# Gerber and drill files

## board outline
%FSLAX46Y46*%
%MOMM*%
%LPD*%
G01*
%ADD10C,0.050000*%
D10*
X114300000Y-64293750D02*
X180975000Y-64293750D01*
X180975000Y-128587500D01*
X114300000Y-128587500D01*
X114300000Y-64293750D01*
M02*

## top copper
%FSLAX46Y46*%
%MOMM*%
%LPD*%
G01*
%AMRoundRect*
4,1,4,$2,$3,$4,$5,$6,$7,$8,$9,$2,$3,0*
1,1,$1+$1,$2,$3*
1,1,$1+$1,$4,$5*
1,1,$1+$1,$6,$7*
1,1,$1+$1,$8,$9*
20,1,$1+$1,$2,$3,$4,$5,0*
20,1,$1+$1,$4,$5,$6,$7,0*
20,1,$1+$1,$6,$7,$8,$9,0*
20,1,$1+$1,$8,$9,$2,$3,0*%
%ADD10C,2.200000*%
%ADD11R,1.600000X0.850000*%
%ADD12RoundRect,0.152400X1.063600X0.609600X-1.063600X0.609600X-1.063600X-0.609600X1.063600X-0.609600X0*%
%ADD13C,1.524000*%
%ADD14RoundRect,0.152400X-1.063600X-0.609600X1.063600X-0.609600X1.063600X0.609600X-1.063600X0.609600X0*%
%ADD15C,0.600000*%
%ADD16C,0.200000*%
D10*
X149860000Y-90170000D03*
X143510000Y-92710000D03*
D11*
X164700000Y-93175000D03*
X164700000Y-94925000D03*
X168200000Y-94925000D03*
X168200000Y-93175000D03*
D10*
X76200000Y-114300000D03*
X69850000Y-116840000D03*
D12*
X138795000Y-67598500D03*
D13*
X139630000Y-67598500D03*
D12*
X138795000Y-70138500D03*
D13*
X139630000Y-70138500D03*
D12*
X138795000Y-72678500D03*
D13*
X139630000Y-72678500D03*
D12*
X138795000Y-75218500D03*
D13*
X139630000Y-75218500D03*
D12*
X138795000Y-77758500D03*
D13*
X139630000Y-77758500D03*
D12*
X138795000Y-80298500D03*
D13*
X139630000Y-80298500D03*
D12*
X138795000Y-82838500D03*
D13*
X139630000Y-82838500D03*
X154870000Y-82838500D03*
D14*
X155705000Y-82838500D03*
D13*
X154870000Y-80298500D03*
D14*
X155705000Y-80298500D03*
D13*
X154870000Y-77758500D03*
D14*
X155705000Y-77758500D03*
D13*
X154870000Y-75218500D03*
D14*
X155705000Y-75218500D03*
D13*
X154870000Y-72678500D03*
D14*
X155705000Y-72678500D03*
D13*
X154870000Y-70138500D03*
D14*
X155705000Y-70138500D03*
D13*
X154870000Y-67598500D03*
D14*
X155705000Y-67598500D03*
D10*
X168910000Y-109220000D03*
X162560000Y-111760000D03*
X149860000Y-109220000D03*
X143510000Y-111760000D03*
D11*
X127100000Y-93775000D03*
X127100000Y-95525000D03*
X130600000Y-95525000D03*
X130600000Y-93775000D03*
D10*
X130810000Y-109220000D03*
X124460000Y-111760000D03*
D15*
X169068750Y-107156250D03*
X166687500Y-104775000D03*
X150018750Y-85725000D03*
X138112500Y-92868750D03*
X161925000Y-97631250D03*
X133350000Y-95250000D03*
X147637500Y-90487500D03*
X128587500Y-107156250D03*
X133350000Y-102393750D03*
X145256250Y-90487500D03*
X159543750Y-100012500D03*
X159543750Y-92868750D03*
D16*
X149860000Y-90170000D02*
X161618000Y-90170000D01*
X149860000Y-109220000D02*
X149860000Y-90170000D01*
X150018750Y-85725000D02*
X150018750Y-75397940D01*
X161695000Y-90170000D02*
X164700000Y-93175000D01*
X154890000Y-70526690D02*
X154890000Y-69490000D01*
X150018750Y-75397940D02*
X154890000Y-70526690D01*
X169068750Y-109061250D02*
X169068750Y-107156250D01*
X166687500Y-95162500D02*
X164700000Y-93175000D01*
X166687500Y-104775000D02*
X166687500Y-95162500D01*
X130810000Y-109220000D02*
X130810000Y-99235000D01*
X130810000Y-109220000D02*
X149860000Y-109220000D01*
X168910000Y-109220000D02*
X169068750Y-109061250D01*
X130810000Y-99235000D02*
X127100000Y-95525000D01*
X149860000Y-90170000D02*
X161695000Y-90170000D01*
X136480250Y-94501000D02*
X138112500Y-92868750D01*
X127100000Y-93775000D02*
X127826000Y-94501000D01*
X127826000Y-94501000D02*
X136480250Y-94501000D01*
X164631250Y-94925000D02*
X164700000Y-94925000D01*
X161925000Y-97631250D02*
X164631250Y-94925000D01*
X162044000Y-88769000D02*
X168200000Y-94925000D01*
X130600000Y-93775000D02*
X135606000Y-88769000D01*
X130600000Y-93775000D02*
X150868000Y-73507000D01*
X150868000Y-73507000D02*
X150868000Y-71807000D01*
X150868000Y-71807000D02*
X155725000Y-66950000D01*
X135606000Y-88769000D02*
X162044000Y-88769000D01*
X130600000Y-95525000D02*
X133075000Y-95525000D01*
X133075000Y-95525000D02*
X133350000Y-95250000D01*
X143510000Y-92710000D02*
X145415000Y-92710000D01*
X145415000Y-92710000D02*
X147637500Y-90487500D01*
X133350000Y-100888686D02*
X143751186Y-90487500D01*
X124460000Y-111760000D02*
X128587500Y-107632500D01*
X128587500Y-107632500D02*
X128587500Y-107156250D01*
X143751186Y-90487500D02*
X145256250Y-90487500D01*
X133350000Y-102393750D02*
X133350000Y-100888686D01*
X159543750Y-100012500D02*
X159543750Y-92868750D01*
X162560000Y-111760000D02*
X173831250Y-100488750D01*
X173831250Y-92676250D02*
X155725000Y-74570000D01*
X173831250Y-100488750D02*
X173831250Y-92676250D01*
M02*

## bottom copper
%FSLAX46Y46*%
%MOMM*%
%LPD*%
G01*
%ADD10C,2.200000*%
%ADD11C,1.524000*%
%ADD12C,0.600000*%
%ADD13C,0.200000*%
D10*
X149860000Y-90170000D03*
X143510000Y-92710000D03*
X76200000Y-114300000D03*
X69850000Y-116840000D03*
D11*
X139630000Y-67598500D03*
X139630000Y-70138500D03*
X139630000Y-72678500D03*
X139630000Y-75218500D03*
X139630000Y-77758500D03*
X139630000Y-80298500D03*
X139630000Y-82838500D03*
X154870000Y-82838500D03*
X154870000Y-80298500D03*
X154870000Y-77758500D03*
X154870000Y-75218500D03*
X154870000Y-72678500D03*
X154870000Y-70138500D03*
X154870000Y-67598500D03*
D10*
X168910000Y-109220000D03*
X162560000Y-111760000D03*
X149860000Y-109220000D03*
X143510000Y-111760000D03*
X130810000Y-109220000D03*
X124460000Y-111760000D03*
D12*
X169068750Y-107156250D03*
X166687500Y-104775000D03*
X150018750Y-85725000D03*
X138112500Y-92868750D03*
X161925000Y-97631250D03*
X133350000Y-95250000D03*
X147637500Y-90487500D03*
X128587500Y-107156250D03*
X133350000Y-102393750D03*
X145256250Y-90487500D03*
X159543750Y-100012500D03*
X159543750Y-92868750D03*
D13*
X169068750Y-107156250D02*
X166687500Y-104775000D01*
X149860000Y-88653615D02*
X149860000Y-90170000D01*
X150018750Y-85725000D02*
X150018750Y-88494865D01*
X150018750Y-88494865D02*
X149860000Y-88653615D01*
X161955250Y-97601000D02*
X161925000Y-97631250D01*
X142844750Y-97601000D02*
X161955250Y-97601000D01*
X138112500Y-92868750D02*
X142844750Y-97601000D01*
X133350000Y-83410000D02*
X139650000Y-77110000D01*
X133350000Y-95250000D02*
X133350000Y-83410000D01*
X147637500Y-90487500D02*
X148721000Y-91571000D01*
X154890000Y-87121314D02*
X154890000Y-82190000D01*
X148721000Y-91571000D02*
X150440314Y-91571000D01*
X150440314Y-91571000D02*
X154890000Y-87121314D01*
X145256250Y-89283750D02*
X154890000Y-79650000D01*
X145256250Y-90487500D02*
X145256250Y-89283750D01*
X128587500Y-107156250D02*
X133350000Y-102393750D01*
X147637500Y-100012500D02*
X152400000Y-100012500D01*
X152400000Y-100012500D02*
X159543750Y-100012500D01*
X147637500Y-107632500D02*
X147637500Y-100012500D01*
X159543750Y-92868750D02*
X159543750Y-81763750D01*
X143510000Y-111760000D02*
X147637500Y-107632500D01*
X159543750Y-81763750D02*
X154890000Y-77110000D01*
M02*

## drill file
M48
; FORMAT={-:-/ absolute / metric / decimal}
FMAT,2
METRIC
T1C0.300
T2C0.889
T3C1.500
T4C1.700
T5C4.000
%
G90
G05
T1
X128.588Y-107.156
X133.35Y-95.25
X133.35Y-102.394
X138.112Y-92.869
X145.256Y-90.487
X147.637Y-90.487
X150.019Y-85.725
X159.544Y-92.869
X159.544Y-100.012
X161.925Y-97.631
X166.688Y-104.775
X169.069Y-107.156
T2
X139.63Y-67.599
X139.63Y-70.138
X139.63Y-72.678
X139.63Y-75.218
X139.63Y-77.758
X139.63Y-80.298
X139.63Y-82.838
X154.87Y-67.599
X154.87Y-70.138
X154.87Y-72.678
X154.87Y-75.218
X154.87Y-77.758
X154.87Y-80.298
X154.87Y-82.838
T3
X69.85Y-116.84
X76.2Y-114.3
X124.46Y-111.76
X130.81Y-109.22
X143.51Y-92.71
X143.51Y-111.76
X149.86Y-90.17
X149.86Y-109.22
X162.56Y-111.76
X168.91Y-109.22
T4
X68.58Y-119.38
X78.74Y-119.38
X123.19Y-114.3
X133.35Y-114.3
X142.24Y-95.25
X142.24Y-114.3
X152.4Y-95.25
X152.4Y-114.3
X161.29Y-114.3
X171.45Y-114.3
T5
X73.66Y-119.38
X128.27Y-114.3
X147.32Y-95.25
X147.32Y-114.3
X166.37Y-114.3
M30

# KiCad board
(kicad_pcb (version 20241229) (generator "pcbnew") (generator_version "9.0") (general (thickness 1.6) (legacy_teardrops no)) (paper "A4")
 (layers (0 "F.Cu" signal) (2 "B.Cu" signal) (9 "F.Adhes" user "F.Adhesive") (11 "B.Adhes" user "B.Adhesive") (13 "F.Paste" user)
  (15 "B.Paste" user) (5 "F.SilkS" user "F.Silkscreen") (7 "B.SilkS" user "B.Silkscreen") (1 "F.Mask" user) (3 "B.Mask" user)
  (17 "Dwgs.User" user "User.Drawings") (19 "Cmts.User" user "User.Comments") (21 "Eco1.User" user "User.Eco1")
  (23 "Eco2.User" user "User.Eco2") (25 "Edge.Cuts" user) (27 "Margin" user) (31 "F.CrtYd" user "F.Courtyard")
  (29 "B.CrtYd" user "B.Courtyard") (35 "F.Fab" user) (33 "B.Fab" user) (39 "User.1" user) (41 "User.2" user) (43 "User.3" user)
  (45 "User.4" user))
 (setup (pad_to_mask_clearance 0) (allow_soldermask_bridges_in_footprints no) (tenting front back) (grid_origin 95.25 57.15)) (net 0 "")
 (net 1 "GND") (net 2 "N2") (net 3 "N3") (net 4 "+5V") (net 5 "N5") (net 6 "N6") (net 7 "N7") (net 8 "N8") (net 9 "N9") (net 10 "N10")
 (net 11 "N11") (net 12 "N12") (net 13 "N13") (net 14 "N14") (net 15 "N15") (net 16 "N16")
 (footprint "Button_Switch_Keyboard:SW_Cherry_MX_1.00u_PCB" (layer "F.Cu") (at 149.86 90.17)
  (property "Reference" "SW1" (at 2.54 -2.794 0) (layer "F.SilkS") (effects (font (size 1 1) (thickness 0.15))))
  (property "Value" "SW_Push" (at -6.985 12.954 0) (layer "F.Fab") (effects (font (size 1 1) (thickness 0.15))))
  (pad "" np_thru_hole circle (at -7.62 5.08) (size 1.7 1.7) (drill 1.7) (layers "*.Cu" "*.Mask"))
  (pad "" np_thru_hole circle (at -2.54 5.08) (size 4 4) (drill 4) (layers "*.Cu" "*.Mask"))
  (pad "" np_thru_hole circle (at 2.54 5.08) (size 1.7 1.7) (drill 1.7) (layers "*.Cu" "*.Mask"))
  (pad "1" thru_hole circle (at 0 0) (size 2.2 2.2) (drill 1.5) (layers "*.Cu" "*.Mask") (remove_unused_layers no) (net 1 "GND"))
  (pad "2" thru_hole circle (at -6.35 2.54) (size 2.2 2.2) (drill 1.5) (layers "*.Cu" "*.Mask") (remove_unused_layers no) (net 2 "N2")))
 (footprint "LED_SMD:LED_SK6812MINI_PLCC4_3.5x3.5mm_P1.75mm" (layer "F.Cu") (at 166.45 94.05)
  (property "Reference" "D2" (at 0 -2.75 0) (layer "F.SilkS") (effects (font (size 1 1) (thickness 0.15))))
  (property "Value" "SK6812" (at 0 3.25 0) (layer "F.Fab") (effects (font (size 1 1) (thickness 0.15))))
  (pad "1" smd rect (at -1.75 -0.875) (size 1.6 0.85) (layers "F.Cu" "F.Mask" "F.Paste") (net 1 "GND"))
  (pad "2" smd rect (at -1.75 0.875) (size 1.6 0.85) (layers "F.Cu" "F.Mask" "F.Paste") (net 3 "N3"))
  (pad "3" smd rect (at 1.75 0.875) (size 1.6 0.85) (layers "F.Cu" "F.Mask" "F.Paste") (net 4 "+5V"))
  (pad "4" smd rect (at 1.75 -0.875) (size 1.6 0.85) (layers "F.Cu" "F.Mask" "F.Paste") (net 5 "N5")))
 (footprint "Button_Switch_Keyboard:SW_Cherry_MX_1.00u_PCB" (layer "F.Cu") (at 76.2 114.3)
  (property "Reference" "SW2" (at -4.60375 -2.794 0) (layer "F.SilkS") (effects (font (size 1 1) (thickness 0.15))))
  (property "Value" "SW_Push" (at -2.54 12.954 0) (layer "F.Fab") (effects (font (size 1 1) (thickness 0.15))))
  (pad "" np_thru_hole circle (at -7.62 5.08) (size 1.7 1.7) (drill 1.7) (layers "*.Cu" "*.Mask"))
  (pad "" np_thru_hole circle (at -2.54 5.08) (size 4 4) (drill 4) (layers "*.Cu" "*.Mask"))
  (pad "" np_thru_hole circle (at 2.54 5.08) (size 1.7 1.7) (drill 1.7) (layers "*.Cu" "*.Mask"))
  (pad "1" thru_hole circle (at 0 0) (size 2.2 2.2) (drill 1.5) (layers "*.Cu" "*.Mask") (remove_unused_layers no))
  (pad "2" thru_hole circle (at -6.35 2.54) (size 2.2 2.2) (drill 1.5) (layers "*.Cu" "*.Mask") (remove_unused_layers no)))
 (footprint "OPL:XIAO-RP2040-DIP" (layer "F.Cu") (at 147.25 75.2185)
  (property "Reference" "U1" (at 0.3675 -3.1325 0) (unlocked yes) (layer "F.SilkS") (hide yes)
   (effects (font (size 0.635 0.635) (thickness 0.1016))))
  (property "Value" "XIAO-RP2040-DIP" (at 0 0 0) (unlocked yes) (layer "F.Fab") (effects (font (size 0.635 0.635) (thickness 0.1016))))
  (pad "1" smd roundrect (at -8.455 -7.62 180) (size 2.432 1.524) (layers "F.Cu" "F.Mask") (roundrect_rratio 0.1) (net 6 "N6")
   (thermal_bridge_angle 45))
  (pad "1" thru_hole circle (at -7.62 -7.62 180) (size 1.524 1.524) (drill 0.889) (layers "*.Cu" "*.Mask") (remove_unused_layers no)
   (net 6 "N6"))
  (pad "2" smd roundrect (at -8.455 -5.08 180) (size 2.432 1.524) (layers "F.Cu" "F.Mask") (roundrect_rratio 0.1) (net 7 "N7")
   (thermal_bridge_angle 45))
  (pad "2" thru_hole circle (at -7.62 -5.08 180) (size 1.524 1.524) (drill 0.889) (layers "*.Cu" "*.Mask") (remove_unused_layers no)
   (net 7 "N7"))
  (pad "3" smd roundrect (at -8.455 -2.54 180) (size 2.432 1.524) (layers "F.Cu" "F.Mask") (roundrect_rratio 0.1) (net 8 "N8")
   (thermal_bridge_angle 45))
  (pad "3" thru_hole circle (at -7.62 -2.54 180) (size 1.524 1.524) (drill 0.889) (layers "*.Cu" "*.Mask") (remove_unused_layers no)
   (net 8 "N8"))
  (pad "4" smd roundrect (at -8.455 0 180) (size 2.432 1.524) (layers "F.Cu" "F.Mask") (roundrect_rratio 0.1) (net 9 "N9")
   (thermal_bridge_angle 45))
  (pad "4" thru_hole circle (at -7.62 0 180) (size 1.524 1.524) (drill 0.889) (layers "*.Cu" "*.Mask") (remove_unused_layers no)
   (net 9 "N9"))
  (pad "5" smd roundrect (at -8.455 2.54 180) (size 2.432 1.524) (layers "F.Cu" "F.Mask") (roundrect_rratio 0.1) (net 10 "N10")
   (thermal_bridge_angle 45))
  (pad "5" thru_hole circle (at -7.62 2.54 180) (size 1.524 1.524) (drill 0.889) (layers "*.Cu" "*.Mask") (remove_unused_layers no)
   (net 10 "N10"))
  (pad "6" smd roundrect (at -8.455 5.08 180) (size 2.432 1.524) (layers "F.Cu" "F.Mask") (roundrect_rratio 0.1) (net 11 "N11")
   (thermal_bridge_angle 45))
  (pad "6" thru_hole circle (at -7.62 5.08 180) (size 1.524 1.524) (drill 0.889) (layers "*.Cu" "*.Mask") (remove_unused_layers no)
   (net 11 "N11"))
  (pad "7" smd roundrect (at -8.455 7.62 180) (size 2.432 1.524) (layers "F.Cu" "F.Mask") (roundrect_rratio 0.1) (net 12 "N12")
   (thermal_bridge_angle 45))
  (pad "7" thru_hole circle (at -7.62 7.62 180) (size 1.524 1.524) (drill 0.889) (layers "*.Cu" "*.Mask") (remove_unused_layers no)
   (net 12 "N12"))
  (pad "8" thru_hole circle (at 7.62 7.62) (size 1.524 1.524) (drill 0.889) (layers "*.Cu" "*.Mask") (remove_unused_layers no) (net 2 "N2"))
  (pad "8" smd roundrect (at 8.455 7.62) (size 2.432 1.524) (layers "F.Cu" "F.Mask") (roundrect_rratio 0.1) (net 2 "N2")
   (thermal_bridge_angle 45))
  (pad "9" thru_hole circle (at 7.62 5.08) (size 1.524 1.524) (drill 0.889) (layers "*.Cu" "*.Mask") (remove_unused_layers no)
   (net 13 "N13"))
  (pad "9" smd roundrect (at 8.455 5.08) (size 2.432 1.524) (layers "F.Cu" "F.Mask") (roundrect_rratio 0.1) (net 13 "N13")
   (thermal_bridge_angle 45))
  (pad "10" thru_hole circle (at 7.62 2.54) (size 1.524 1.524) (drill 0.889) (layers "*.Cu" "*.Mask") (remove_unused_layers no)
   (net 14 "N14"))
  (pad "10" smd roundrect (at 8.455 2.54) (size 2.432 1.524) (layers "F.Cu" "F.Mask") (roundrect_rratio 0.1) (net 14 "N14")
   (thermal_bridge_angle 45))
  (pad "11" thru_hole circle (at 7.62 0) (size 1.524 1.524) (drill 0.889) (layers "*.Cu" "*.Mask") (remove_unused_layers no) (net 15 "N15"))
  (pad "11" smd roundrect (at 8.455 0) (size 2.432 1.524) (layers "F.Cu" "F.Mask") (roundrect_rratio 0.1) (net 15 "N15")
   (thermal_bridge_angle 45))
  (pad "12" thru_hole circle (at 7.62 -2.54) (size 1.524 1.524) (drill 0.889) (layers "*.Cu" "*.Mask") (remove_unused_layers no)
   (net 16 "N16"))
  (pad "12" smd roundrect (at 8.455 -2.54) (size 2.432 1.524) (layers "F.Cu" "F.Mask") (roundrect_rratio 0.1) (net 16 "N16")
   (thermal_bridge_angle 45))
  (pad "13" thru_hole circle (at 7.62 -5.08) (size 1.524 1.524) (drill 0.889) (layers "*.Cu" "*.Mask") (remove_unused_layers no)
   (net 1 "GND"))
  (pad "13" smd roundrect (at 8.455 -5.08) (size 2.432 1.524) (layers "F.Cu" "F.Mask") (roundrect_rratio 0.1) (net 1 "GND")
   (thermal_bridge_angle 45))
  (pad "14" thru_hole circle (at 7.62 -7.62) (size 1.524 1.524) (drill 0.889) (layers "*.Cu" "*.Mask") (remove_unused_layers no)
   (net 4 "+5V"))
  (pad "14" smd roundrect (at 8.455 -7.62) (size 2.432 1.524) (layers "F.Cu" "F.Mask") (roundrect_rratio 0.1) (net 4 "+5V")
   (thermal_bridge_angle 45)))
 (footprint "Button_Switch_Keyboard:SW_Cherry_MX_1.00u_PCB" (layer "F.Cu") (at 168.91 109.22)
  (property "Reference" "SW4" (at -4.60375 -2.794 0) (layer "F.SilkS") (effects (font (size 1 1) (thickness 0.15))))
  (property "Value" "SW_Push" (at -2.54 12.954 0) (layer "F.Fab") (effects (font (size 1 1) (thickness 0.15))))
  (pad "" np_thru_hole circle (at -7.62 5.08) (size 1.7 1.7) (drill 1.7) (layers "*.Cu" "*.Mask"))
  (pad "" np_thru_hole circle (at -2.54 5.08) (size 4 4) (drill 4) (layers "*.Cu" "*.Mask"))
  (pad "" np_thru_hole circle (at 2.54 5.08) (size 1.7 1.7) (drill 1.7) (layers "*.Cu" "*.Mask"))
  (pad "1" thru_hole circle (at 0 0) (size 2.2 2.2) (drill 1.5) (layers "*.Cu" "*.Mask") (remove_unused_layers no) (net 1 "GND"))
  (pad "2" thru_hole circle (at -6.35 2.54) (size 2.2 2.2) (drill 1.5) (layers "*.Cu" "*.Mask") (remove_unused_layers no) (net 15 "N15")))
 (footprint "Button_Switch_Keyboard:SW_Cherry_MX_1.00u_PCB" (layer "F.Cu") (at 149.86 109.22)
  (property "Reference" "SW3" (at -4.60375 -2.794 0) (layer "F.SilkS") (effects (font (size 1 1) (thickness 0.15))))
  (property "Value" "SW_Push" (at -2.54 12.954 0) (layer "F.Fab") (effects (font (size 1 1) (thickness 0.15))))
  (pad "" np_thru_hole circle (at -7.62 5.08) (size 1.7 1.7) (drill 1.7) (layers "*.Cu" "*.Mask"))
  (pad "" np_thru_hole circle (at -2.54 5.08) (size 4 4) (drill 4) (layers "*.Cu" "*.Mask"))
  (pad "" np_thru_hole circle (at 2.54 5.08) (size 1.7 1.7) (drill 1.7) (layers "*.Cu" "*.Mask"))
  (pad "1" thru_hole circle (at 0 0) (size 2.2 2.2) (drill 1.5) (layers "*.Cu" "*.Mask") (remove_unused_layers no) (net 1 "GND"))
  (pad "2" thru_hole circle (at -6.35 2.54) (size 2.2 2.2) (drill 1.5) (layers "*.Cu" "*.Mask") (remove_unused_layers no) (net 14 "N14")))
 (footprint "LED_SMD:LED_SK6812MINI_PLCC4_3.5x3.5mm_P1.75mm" (layer "F.Cu") (at 128.85 94.65)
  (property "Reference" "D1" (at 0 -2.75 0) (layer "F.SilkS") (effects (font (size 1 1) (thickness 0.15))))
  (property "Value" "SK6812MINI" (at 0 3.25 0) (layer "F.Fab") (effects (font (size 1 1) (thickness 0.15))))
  (pad "1" smd rect (at -1.75 -0.875) (size 1.6 0.85) (layers "F.Cu" "F.Mask" "F.Paste") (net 3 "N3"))
  (pad "2" smd rect (at -1.75 0.875) (size 1.6 0.85) (layers "F.Cu" "F.Mask" "F.Paste") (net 1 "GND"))
  (pad "3" smd rect (at 1.75 0.875) (size 1.6 0.85) (layers "F.Cu" "F.Mask" "F.Paste") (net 10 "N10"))
  (pad "4" smd rect (at 1.75 -0.875) (size 1.6 0.85) (layers "F.Cu" "F.Mask" "F.Paste") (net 4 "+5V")))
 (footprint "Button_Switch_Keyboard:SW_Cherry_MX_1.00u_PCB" (layer "F.Cu") (at 130.81 109.22)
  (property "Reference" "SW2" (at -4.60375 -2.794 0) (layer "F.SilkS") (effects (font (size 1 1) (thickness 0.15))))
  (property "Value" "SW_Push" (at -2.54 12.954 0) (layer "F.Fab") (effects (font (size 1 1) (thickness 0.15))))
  (pad "" np_thru_hole circle (at -7.62 5.08) (size 1.7 1.7) (drill 1.7) (layers "*.Cu" "*.Mask"))
  (pad "" np_thru_hole circle (at -2.54 5.08) (size 4 4) (drill 4) (layers "*.Cu" "*.Mask"))
  (pad "" np_thru_hole circle (at 2.54 5.08) (size 1.7 1.7) (drill 1.7) (layers "*.Cu" "*.Mask"))
  (pad "1" thru_hole circle (at 0 0) (size 2.2 2.2) (drill 1.5) (layers "*.Cu" "*.Mask") (remove_unused_layers no) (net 1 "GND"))
  (pad "2" thru_hole circle (at -6.35 2.54) (size 2.2 2.2) (drill 1.5) (layers "*.Cu" "*.Mask") (remove_unused_layers no) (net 13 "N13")))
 (gr_rect (start 114.3 64.29375) (end 180.975 128.5875) (stroke (width 0.05) (type default)) (fill no) (layer "Edge.Cuts"))
 (segment (start 149.86 90.17) (end 161.618 90.17) (width 0.2) (layer "F.Cu") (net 1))
 (segment (start 149.86 109.22) (end 149.86 90.17) (width 0.2) (layer "F.Cu") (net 1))
 (segment (start 150.01875 85.725) (end 150.01875 75.39794) (width 0.2) (layer "F.Cu") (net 1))
 (segment (start 161.695 90.17) (end 164.7 93.175) (width 0.2) (layer "F.Cu") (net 1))
 (segment (start 154.89 70.52669) (end 154.89 69.49) (width 0.2) (layer "F.Cu") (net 1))
 (segment (start 150.01875 75.39794) (end 154.89 70.52669) (width 0.2) (layer "F.Cu") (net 1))
 (segment (start 169.06875 109.06125) (end 169.06875 107.15625) (width 0.2) (layer "F.Cu") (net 1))
 (segment (start 166.6875 95.1625) (end 164.7 93.175) (width 0.2) (layer "F.Cu") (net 1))
 (segment (start 166.6875 104.775) (end 166.6875 95.1625) (width 0.2) (layer "F.Cu") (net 1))
 (segment (start 130.81 109.22) (end 130.81 99.235) (width 0.2) (layer "F.Cu") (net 1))
 (segment (start 130.81 109.22) (end 149.86 109.22) (width 0.2) (layer "F.Cu") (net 1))
 (segment (start 168.91 109.22) (end 169.06875 109.06125) (width 0.2) (layer "F.Cu") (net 1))
 (segment (start 130.81 99.235) (end 127.1 95.525) (width 0.2) (layer "F.Cu") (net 1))
 (segment (start 149.86 90.17) (end 161.695 90.17) (width 0.2) (layer "F.Cu") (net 1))
 (via (at 169.06875 107.15625) (size 0.6) (drill 0.3) (layers "F.Cu" "B.Cu") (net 1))
 (via (at 166.6875 104.775) (size 0.6) (drill 0.3) (layers "F.Cu" "B.Cu") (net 1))
 (via (at 150.01875 85.725) (size 0.6) (drill 0.3) (layers "F.Cu" "B.Cu") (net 1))
 (segment (start 169.06875 107.15625) (end 166.6875 104.775) (width 0.2) (layer "B.Cu") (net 1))
 (segment (start 149.86 88.653615) (end 149.86 90.17) (width 0.2) (layer "B.Cu") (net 1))
 (segment (start 150.01875 85.725) (end 150.01875 88.494865) (width 0.2) (layer "B.Cu") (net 1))
 (segment (start 150.01875 88.494865) (end 149.86 88.653615) (width 0.2) (layer "B.Cu") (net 1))
 (segment (start 136.48025 94.501) (end 138.1125 92.86875) (width 0.2) (layer "F.Cu") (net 3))
 (segment (start 127.1 93.775) (end 127.826 94.501) (width 0.2) (layer "F.Cu") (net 3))
 (segment (start 127.826 94.501) (end 136.48025 94.501) (width 0.2) (layer "F.Cu") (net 3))
 (segment (start 164.63125 94.925) (end 164.7 94.925) (width 0.2) (layer "F.Cu") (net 3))
 (segment (start 161.925 97.63125) (end 164.63125 94.925) (width 0.2) (layer "F.Cu") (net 3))
 (via (at 138.1125 92.86875) (size 0.6) (drill 0.3) (layers "F.Cu" "B.Cu") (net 3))
 (via (at 161.925 97.63125) (size 0.6) (drill 0.3) (layers "F.Cu" "B.Cu") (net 3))
 (segment (start 161.95525 97.601) (end 161.925 97.63125) (width 0.2) (layer "B.Cu") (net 3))
 (segment (start 142.84475 97.601) (end 161.95525 97.601) (width 0.2) (layer "B.Cu") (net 3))
 (segment (start 138.1125 92.86875) (end 142.84475 97.601) (width 0.2) (layer "B.Cu") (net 3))
 (segment (start 162.044 88.769) (end 168.2 94.925) (width 0.2) (layer "F.Cu") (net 4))
 (segment (start 130.6 93.775) (end 135.606 88.769) (width 0.2) (layer "F.Cu") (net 4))
 (segment (start 130.6 93.775) (end 150.868 73.507) (width 0.2) (layer "F.Cu") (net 4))
 (segment (start 150.868 73.507) (end 150.868 71.807) (width 0.2) (layer "F.Cu") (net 4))
 (segment (start 150.868 71.807) (end 155.725 66.95) (width 0.2) (layer "F.Cu") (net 4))
 (segment (start 135.606 88.769) (end 162.044 88.769) (width 0.2) (layer "F.Cu") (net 4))
 (segment (start 130.6 95.525) (end 133.075 95.525) (width 0.2) (layer "F.Cu") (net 10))
 (segment (start 133.075 95.525) (end 133.35 95.25) (width 0.2) (layer "F.Cu") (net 10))
 (via (at 133.35 95.25) (size 0.6) (drill 0.3) (layers "F.Cu" "B.Cu") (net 10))
 (segment (start 133.35 83.41) (end 139.65 77.11) (width 0.2) (layer "B.Cu") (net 10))
 (segment (start 133.35 95.25) (end 133.35 83.41) (width 0.2) (layer "B.Cu") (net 10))
 (segment (start 143.51 92.71) (end 145.415 92.71) (width 0.2) (layer "F.Cu") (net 2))
 (segment (start 145.415 92.71) (end 147.6375 90.4875) (width 0.2) (layer "F.Cu") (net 2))
 (via (at 147.6375 90.4875) (size 0.6) (drill 0.3) (layers "F.Cu" "B.Cu") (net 2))
 (segment (start 147.6375 90.4875) (end 148.721 91.571) (width 0.2) (layer "B.Cu") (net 2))
 (segment (start 154.89 87.121314) (end 154.89 82.19) (width 0.2) (layer "B.Cu") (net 2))
 (segment (start 148.721 91.571) (end 150.440314 91.571) (width 0.2) (layer "B.Cu") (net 2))
 (segment (start 150.440314 91.571) (end 154.89 87.121314) (width 0.2) (layer "B.Cu") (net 2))
 (segment (start 133.35 100.888686) (end 143.751186 90.4875) (width 0.2) (layer "F.Cu") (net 13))
 (segment (start 124.46 111.76) (end 128.5875 107.6325) (width 0.2) (layer "F.Cu") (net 13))
 (segment (start 128.5875 107.6325) (end 128.5875 107.15625) (width 0.2) (layer "F.Cu") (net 13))
 (segment (start 143.751186 90.4875) (end 145.25625 90.4875) (width 0.2) (layer "F.Cu") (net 13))
 (segment (start 133.35 102.39375) (end 133.35 100.888686) (width 0.2) (layer "F.Cu") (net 13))
 (via (at 128.5875 107.15625) (size 0.6) (drill 0.3) (layers "F.Cu" "B.Cu") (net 13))
 (via (at 133.35 102.39375) (size 0.6) (drill 0.3) (layers "F.Cu" "B.Cu") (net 13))
 (via (at 145.25625 90.4875) (size 0.6) (drill 0.3) (layers "F.Cu" "B.Cu") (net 13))
 (segment (start 145.25625 89.28375) (end 154.89 79.65) (width 0.2) (layer "B.Cu") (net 13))
 (segment (start 145.25625 90.4875) (end 145.25625 89.28375) (width 0.2) (layer "B.Cu") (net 13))
 (segment (start 128.5875 107.15625) (end 133.35 102.39375) (width 0.2) (layer "B.Cu") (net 13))
 (segment (start 159.54375 100.0125) (end 159.54375 92.86875) (width 0.2) (layer "F.Cu") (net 14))
 (via (at 159.54375 100.0125) (size 0.6) (drill 0.3) (layers "F.Cu" "B.Cu") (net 14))
 (via (at 159.54375 92.86875) (size 0.6) (drill 0.3) (layers "F.Cu" "B.Cu") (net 14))
 (segment (start 147.6375 100.0125) (end 152.4 100.0125) (width 0.2) (layer "B.Cu") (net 14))
 (segment (start 152.4 100.0125) (end 159.54375 100.0125) (width 0.2) (layer "B.Cu") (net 14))
 (segment (start 147.6375 107.6325) (end 147.6375 100.0125) (width 0.2) (layer "B.Cu") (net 14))
 (segment (start 159.54375 92.86875) (end 159.54375 81.76375) (width 0.2) (layer "B.Cu") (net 14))
 (segment (start 143.51 111.76) (end 147.6375 107.6325) (width 0.2) (layer "B.Cu") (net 14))
 (segment (start 159.54375 81.76375) (end 154.89 77.11) (width 0.2) (layer "B.Cu") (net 14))
 (segment (start 162.56 111.76) (end 173.83125 100.48875) (width 0.2) (layer "F.Cu") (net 15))
 (segment (start 173.83125 92.67625) (end 155.725 74.57) (width 0.2) (layer "F.Cu") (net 15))
 (segment (start 173.83125 100.48875) (end 173.83125 92.67625) (width 0.2) (layer "F.Cu") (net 15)))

